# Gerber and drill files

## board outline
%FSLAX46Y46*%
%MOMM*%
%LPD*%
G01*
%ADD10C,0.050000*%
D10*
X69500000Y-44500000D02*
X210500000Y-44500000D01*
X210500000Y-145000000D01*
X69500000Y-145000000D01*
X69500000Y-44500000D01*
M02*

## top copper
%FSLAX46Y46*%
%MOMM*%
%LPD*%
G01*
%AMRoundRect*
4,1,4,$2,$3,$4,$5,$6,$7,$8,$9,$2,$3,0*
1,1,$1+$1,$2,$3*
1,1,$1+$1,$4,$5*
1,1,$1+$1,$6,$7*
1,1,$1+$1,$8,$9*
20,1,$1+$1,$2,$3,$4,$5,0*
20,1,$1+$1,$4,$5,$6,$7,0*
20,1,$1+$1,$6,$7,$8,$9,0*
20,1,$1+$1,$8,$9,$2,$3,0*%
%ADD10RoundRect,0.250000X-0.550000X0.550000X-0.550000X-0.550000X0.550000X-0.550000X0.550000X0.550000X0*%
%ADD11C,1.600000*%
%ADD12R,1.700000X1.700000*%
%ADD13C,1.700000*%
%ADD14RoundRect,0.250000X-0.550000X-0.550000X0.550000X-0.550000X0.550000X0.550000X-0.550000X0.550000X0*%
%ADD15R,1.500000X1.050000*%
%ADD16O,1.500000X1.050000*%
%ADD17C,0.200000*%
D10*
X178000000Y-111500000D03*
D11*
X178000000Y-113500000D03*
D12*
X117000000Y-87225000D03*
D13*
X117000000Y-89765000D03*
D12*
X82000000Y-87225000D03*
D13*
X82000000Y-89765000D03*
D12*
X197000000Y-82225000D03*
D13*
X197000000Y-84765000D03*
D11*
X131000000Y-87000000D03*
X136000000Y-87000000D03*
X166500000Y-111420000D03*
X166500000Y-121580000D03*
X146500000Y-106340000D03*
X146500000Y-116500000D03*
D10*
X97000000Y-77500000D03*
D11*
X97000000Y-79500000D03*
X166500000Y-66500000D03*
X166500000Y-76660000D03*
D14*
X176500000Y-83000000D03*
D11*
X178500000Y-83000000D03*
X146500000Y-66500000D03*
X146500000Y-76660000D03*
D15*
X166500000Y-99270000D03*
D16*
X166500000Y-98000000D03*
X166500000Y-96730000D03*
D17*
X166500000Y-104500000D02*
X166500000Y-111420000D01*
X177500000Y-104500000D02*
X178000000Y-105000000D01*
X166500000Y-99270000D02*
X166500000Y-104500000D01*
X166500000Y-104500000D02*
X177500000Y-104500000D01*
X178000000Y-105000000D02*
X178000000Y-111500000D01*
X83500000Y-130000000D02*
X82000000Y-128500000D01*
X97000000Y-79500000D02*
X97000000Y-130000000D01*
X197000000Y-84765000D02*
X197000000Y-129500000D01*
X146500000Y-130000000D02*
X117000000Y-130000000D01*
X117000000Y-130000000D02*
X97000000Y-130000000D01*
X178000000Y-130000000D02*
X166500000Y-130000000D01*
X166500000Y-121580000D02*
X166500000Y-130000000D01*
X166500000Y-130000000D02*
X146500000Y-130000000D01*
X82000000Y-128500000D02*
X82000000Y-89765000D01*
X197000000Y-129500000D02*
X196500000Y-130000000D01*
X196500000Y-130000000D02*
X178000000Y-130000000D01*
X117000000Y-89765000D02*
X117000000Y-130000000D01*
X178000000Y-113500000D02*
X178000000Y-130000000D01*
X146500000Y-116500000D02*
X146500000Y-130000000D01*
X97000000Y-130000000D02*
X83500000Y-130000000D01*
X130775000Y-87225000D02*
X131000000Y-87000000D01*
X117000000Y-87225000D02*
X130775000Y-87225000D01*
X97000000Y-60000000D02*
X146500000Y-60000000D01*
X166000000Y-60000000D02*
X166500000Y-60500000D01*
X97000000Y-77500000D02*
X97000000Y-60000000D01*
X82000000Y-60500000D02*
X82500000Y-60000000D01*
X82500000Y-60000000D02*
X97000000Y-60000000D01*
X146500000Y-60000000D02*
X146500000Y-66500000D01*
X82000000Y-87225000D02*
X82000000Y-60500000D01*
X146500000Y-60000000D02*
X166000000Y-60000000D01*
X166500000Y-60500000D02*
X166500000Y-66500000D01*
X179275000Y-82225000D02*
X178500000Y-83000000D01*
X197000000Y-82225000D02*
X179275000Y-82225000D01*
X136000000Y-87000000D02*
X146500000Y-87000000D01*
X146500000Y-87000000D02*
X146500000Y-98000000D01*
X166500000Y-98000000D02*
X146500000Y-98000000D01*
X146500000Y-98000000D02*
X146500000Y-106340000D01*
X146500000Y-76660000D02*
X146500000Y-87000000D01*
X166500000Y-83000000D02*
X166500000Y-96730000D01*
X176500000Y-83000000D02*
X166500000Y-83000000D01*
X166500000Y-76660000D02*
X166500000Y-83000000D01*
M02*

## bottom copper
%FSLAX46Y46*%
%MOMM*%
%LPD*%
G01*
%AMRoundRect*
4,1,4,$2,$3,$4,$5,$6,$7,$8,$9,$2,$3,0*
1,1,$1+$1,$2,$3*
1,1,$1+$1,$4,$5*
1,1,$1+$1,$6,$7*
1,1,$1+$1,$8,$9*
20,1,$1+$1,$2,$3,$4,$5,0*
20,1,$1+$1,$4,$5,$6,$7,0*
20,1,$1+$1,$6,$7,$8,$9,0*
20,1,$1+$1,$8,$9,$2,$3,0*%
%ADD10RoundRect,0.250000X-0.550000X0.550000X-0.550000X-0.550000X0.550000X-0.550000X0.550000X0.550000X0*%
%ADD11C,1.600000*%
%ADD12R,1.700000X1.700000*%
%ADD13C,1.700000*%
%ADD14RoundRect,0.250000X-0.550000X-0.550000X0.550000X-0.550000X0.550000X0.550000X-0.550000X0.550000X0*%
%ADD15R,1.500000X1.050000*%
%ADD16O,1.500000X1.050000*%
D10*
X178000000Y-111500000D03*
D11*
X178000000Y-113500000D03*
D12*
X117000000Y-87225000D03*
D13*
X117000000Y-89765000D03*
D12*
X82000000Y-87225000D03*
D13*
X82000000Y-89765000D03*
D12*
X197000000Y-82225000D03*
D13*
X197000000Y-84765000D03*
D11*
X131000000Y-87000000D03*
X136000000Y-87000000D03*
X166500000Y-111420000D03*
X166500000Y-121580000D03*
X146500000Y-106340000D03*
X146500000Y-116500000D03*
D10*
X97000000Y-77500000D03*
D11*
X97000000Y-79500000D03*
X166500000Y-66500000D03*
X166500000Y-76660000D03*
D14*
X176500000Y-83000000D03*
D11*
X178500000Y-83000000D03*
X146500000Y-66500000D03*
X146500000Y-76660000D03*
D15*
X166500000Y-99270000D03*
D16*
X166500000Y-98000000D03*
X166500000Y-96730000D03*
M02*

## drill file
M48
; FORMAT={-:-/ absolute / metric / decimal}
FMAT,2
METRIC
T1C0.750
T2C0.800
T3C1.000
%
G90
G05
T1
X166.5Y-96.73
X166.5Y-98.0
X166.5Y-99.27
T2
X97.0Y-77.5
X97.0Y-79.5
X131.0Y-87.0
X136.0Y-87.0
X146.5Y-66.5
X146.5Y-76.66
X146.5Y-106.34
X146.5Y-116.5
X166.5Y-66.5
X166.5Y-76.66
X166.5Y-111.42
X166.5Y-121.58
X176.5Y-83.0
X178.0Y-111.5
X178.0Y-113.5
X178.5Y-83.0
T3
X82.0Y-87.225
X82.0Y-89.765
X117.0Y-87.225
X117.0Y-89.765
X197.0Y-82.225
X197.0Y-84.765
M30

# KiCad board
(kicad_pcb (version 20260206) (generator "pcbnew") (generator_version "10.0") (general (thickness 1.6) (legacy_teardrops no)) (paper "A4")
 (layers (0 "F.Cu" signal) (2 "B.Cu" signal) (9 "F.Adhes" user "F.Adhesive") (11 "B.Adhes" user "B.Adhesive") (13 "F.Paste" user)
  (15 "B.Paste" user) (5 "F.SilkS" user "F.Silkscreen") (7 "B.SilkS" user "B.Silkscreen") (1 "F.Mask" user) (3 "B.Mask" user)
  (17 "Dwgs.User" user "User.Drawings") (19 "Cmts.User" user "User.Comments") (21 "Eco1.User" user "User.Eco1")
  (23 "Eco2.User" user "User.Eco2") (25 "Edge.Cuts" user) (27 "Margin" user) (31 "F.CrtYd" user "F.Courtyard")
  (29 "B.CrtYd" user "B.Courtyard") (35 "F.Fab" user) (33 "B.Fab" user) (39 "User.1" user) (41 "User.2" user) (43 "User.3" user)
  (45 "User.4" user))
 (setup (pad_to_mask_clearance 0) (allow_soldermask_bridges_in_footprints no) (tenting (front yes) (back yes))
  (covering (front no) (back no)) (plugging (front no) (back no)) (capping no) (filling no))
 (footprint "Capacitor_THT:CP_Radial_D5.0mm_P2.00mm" (layer "F.Cu") (at 178 111.5 -90)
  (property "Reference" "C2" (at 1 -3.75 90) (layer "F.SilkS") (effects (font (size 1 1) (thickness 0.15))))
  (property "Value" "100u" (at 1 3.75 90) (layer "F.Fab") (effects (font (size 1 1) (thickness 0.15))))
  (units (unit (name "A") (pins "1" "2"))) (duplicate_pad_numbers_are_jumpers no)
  (pad "1" thru_hole roundrect (at 0 0 270) (size 1.6 1.6) (drill 0.8) (layers "*.Cu" "*.Mask") (remove_unused_layers no)
   (roundrect_rratio 0.15625) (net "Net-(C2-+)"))
  (pad "2" thru_hole circle (at 2 0 270) (size 1.6 1.6) (drill 0.8) (layers "*.Cu" "*.Mask") (remove_unused_layers no) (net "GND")))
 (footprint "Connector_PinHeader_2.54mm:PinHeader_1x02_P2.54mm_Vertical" (layer "F.Cu") (at 117 87.225)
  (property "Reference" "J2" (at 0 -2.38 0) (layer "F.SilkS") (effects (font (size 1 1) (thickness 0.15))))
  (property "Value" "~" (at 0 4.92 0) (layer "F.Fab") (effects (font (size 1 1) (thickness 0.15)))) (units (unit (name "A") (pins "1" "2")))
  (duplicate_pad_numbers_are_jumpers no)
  (pad "1" thru_hole rect (at 0 0) (size 1.7 1.7) (drill 1) (layers "*.Cu" "*.Mask") (remove_unused_layers no) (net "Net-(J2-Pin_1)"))
  (pad "2" thru_hole circle (at 0 2.54) (size 1.7 1.7) (drill 1) (layers "*.Cu" "*.Mask") (remove_unused_layers no) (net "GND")))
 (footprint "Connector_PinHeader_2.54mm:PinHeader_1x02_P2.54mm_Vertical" (layer "F.Cu") (at 82 87.225)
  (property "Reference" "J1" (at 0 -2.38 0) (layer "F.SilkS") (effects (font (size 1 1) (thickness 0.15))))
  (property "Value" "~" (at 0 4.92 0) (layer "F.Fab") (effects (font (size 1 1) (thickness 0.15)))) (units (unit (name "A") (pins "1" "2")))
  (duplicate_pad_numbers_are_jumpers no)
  (pad "1" thru_hole rect (at 0 0) (size 1.7 1.7) (drill 1) (layers "*.Cu" "*.Mask") (remove_unused_layers no) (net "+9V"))
  (pad "2" thru_hole circle (at 0 2.54) (size 1.7 1.7) (drill 1) (layers "*.Cu" "*.Mask") (remove_unused_layers no) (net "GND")))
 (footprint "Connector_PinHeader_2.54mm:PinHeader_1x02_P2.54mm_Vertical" (layer "F.Cu") (at 197 82.225)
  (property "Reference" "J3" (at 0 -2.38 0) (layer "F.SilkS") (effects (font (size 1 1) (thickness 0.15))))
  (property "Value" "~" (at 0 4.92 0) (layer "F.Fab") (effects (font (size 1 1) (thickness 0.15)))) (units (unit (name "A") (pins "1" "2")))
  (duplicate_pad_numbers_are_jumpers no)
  (pad "1" thru_hole rect (at 0 0) (size 1.7 1.7) (drill 1) (layers "*.Cu" "*.Mask") (remove_unused_layers no) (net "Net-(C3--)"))
  (pad "2" thru_hole circle (at 0 2.54) (size 1.7 1.7) (drill 1) (layers "*.Cu" "*.Mask") (remove_unused_layers no) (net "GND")))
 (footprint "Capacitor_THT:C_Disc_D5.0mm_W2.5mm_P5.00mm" (layer "F.Cu") (at 131 87)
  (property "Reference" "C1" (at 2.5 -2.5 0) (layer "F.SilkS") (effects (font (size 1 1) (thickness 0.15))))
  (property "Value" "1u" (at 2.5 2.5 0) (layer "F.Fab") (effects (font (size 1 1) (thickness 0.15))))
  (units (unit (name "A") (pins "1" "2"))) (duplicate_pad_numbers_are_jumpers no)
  (pad "1" thru_hole circle (at 0 0) (size 1.6 1.6) (drill 0.8) (layers "*.Cu" "*.Mask") (remove_unused_layers no) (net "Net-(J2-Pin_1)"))
  (pad "2" thru_hole circle (at 5 0) (size 1.6 1.6) (drill 0.8) (layers "*.Cu" "*.Mask") (remove_unused_layers no) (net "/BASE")))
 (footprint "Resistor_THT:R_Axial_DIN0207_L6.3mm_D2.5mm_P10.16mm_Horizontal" (layer "F.Cu") (at 166.5 111.42 -90)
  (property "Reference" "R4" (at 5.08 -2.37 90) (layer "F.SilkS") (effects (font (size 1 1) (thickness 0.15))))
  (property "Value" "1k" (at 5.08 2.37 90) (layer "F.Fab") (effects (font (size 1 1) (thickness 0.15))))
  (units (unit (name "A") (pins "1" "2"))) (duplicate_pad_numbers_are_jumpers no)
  (pad "1" thru_hole circle (at 0 0 270) (size 1.6 1.6) (drill 0.8) (layers "*.Cu" "*.Mask") (remove_unused_layers no) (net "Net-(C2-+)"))
  (pad "2" thru_hole circle (at 10.16 0 270) (size 1.6 1.6) (drill 0.8) (layers "*.Cu" "*.Mask") (remove_unused_layers no) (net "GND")))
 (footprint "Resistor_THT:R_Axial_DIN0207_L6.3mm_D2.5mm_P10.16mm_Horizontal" (layer "F.Cu") (at 146.5 106.34 -90)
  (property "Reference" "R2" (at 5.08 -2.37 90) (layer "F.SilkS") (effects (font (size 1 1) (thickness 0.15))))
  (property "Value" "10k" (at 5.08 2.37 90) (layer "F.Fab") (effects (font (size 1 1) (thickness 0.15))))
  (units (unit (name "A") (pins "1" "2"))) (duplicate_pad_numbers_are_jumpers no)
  (pad "1" thru_hole circle (at 0 0 270) (size 1.6 1.6) (drill 0.8) (layers "*.Cu" "*.Mask") (remove_unused_layers no) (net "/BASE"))
  (pad "2" thru_hole circle (at 10.16 0 270) (size 1.6 1.6) (drill 0.8) (layers "*.Cu" "*.Mask") (remove_unused_layers no) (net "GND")))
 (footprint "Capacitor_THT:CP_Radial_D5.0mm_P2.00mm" (layer "F.Cu") (at 97 77.5 -90)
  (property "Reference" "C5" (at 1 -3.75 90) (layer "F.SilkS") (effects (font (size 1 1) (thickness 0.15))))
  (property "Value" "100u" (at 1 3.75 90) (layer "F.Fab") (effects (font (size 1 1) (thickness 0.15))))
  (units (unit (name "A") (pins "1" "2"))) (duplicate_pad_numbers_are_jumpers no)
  (pad "1" thru_hole roundrect (at 0 0 270) (size 1.6 1.6) (drill 0.8) (layers "*.Cu" "*.Mask") (remove_unused_layers no)
   (roundrect_rratio 0.15625) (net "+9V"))
  (pad "2" thru_hole circle (at 2 0 270) (size 1.6 1.6) (drill 0.8) (layers "*.Cu" "*.Mask") (remove_unused_layers no) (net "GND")))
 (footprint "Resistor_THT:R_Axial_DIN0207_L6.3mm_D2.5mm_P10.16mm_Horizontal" (layer "F.Cu") (at 166.5 66.5 -90)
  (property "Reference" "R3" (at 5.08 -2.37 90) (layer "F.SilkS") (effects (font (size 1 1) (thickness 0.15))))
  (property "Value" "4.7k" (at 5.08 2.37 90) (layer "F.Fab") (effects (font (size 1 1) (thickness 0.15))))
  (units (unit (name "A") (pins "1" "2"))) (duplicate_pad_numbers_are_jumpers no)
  (pad "1" thru_hole circle (at 0 0 270) (size 1.6 1.6) (drill 0.8) (layers "*.Cu" "*.Mask") (remove_unused_layers no) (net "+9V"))
  (pad "2" thru_hole circle (at 10.16 0 270) (size 1.6 1.6) (drill 0.8) (layers "*.Cu" "*.Mask") (remove_unused_layers no)
   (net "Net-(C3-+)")))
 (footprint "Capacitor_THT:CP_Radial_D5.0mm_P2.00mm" (layer "F.Cu") (at 176.5 83)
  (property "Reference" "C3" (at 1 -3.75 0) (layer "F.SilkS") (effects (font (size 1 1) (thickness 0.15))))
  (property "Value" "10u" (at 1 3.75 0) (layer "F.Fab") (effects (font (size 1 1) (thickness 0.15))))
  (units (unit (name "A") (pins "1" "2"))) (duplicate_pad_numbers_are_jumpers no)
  (pad "1" thru_hole roundrect (at 0 0) (size 1.6 1.6) (drill 0.8) (layers "*.Cu" "*.Mask") (remove_unused_layers no)
   (roundrect_rratio 0.15625) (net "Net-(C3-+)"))
  (pad "2" thru_hole circle (at 2 0) (size 1.6 1.6) (drill 0.8) (layers "*.Cu" "*.Mask") (remove_unused_layers no) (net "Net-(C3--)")))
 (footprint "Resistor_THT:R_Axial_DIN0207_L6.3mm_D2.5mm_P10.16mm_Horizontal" (layer "F.Cu") (at 146.5 66.5 -90)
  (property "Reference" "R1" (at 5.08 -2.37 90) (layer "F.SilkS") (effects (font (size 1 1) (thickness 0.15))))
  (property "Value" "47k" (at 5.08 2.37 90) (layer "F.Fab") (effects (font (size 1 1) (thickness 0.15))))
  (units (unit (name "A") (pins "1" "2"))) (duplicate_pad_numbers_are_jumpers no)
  (pad "1" thru_hole circle (at 0 0 270) (size 1.6 1.6) (drill 0.8) (layers "*.Cu" "*.Mask") (remove_unused_layers no) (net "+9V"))
  (pad "2" thru_hole circle (at 10.16 0 270) (size 1.6 1.6) (drill 0.8) (layers "*.Cu" "*.Mask") (remove_unused_layers no) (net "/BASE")))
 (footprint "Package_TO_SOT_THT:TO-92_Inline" (layer "F.Cu") (at 166.5 99.27 90)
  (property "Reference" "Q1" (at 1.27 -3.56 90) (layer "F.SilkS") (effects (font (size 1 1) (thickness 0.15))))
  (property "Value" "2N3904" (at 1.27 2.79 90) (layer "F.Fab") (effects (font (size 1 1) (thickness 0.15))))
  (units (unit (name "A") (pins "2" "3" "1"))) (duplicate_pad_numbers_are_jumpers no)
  (pad "1" thru_hole rect (at 0 0 90) (size 1.05 1.5) (drill 0.75) (layers "*.Cu" "*.Mask") (remove_unused_layers no) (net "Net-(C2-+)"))
  (pad "2" thru_hole oval (at 1.27 0 90) (size 1.05 1.5) (drill 0.75) (layers "*.Cu" "*.Mask") (remove_unused_layers no) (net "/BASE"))
  (pad "3" thru_hole oval (at 2.54 0 90) (size 1.05 1.5) (drill 0.75) (layers "*.Cu" "*.Mask") (remove_unused_layers no) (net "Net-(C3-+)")))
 (gr_rect (start 69.5 44.5) (end 210.5 145) (stroke (width 0.05) (type default)) (fill no) (layer "Edge.Cuts"))
 (segment (start 166.5 104.5) (end 166.5 111.42) (width 0.2) (layer "F.Cu") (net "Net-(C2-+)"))
 (segment (start 177.5 104.5) (end 178 105) (width 0.2) (layer "F.Cu") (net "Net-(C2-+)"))
 (segment (start 166.5 99.27) (end 166.5 104.5) (width 0.2) (layer "F.Cu") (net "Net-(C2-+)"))
 (segment (start 166.5 104.5) (end 177.5 104.5) (width 0.2) (layer "F.Cu") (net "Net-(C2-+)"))
 (segment (start 178 105) (end 178 111.5) (width 0.2) (layer "F.Cu") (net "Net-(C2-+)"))
 (segment (start 83.5 130) (end 82 128.5) (width 0.2) (layer "F.Cu") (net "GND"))
 (segment (start 97 79.5) (end 97 130) (width 0.2) (layer "F.Cu") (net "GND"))
 (segment (start 197 84.765) (end 197 129.5) (width 0.2) (layer "F.Cu") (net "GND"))
 (segment (start 146.5 130) (end 117 130) (width 0.2) (layer "F.Cu") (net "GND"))
 (segment (start 117 130) (end 97 130) (width 0.2) (layer "F.Cu") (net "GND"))
 (segment (start 178 130) (end 166.5 130) (width 0.2) (layer "F.Cu") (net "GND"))
 (segment (start 166.5 121.58) (end 166.5 130) (width 0.2) (layer "F.Cu") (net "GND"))
 (segment (start 166.5 130) (end 146.5 130) (width 0.2) (layer "F.Cu") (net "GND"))
 (segment (start 82 128.5) (end 82 89.765) (width 0.2) (layer "F.Cu") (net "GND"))
 (segment (start 197 129.5) (end 196.5 130) (width 0.2) (layer "F.Cu") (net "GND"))
 (segment (start 196.5 130) (end 178 130) (width 0.2) (layer "F.Cu") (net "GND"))
 (segment (start 117 89.765) (end 117 130) (width 0.2) (layer "F.Cu") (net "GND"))
 (segment (start 178 113.5) (end 178 130) (width 0.2) (layer "F.Cu") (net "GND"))
 (segment (start 146.5 116.5) (end 146.5 130) (width 0.2) (layer "F.Cu") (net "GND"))
 (segment (start 97 130) (end 83.5 130) (width 0.2) (layer "F.Cu") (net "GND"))
 (segment (start 130.775 87.225) (end 131 87) (width 0.2) (layer "F.Cu") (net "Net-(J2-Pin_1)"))
 (segment (start 117 87.225) (end 130.775 87.225) (width 0.2) (layer "F.Cu") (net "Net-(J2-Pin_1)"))
 (segment (start 97 60) (end 146.5 60) (width 0.2) (layer "F.Cu") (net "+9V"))
 (segment (start 166 60) (end 166.5 60.5) (width 0.2) (layer "F.Cu") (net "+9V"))
 (segment (start 97 77.5) (end 97 60) (width 0.2) (layer "F.Cu") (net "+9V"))
 (segment (start 82 60.5) (end 82.5 60) (width 0.2) (layer "F.Cu") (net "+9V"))
 (segment (start 82.5 60) (end 97 60) (width 0.2) (layer "F.Cu") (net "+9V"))
 (segment (start 146.5 60) (end 146.5 66.5) (width 0.2) (layer "F.Cu") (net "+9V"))
 (segment (start 82 87.225) (end 82 60.5) (width 0.2) (layer "F.Cu") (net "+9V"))
 (segment (start 146.5 60) (end 166 60) (width 0.2) (layer "F.Cu") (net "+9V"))
 (segment (start 166.5 60.5) (end 166.5 66.5) (width 0.2) (layer "F.Cu") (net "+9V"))
 (segment (start 179.275 82.225) (end 178.5 83) (width 0.2) (layer "F.Cu") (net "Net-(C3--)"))
 (segment (start 197 82.225) (end 179.275 82.225) (width 0.2) (layer "F.Cu") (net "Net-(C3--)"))
 (segment (start 136 87) (end 146.5 87) (width 0.2) (layer "F.Cu") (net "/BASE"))
 (segment (start 146.5 87) (end 146.5 98) (width 0.2) (layer "F.Cu") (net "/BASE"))
 (segment (start 166.5 98) (end 146.5 98) (width 0.2) (layer "F.Cu") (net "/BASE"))
 (segment (start 146.5 98) (end 146.5 106.34) (width 0.2) (layer "F.Cu") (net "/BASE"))
 (segment (start 146.5 76.66) (end 146.5 87) (width 0.2) (layer "F.Cu") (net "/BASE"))
 (segment (start 166.5 83) (end 166.5 96.73) (width 0.2) (layer "F.Cu") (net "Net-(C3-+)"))
 (segment (start 176.5 83) (end 166.5 83) (width 0.2) (layer "F.Cu") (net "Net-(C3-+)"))
 (segment (start 166.5 76.66) (end 166.5 83) (width 0.2) (layer "F.Cu") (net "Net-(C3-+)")))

